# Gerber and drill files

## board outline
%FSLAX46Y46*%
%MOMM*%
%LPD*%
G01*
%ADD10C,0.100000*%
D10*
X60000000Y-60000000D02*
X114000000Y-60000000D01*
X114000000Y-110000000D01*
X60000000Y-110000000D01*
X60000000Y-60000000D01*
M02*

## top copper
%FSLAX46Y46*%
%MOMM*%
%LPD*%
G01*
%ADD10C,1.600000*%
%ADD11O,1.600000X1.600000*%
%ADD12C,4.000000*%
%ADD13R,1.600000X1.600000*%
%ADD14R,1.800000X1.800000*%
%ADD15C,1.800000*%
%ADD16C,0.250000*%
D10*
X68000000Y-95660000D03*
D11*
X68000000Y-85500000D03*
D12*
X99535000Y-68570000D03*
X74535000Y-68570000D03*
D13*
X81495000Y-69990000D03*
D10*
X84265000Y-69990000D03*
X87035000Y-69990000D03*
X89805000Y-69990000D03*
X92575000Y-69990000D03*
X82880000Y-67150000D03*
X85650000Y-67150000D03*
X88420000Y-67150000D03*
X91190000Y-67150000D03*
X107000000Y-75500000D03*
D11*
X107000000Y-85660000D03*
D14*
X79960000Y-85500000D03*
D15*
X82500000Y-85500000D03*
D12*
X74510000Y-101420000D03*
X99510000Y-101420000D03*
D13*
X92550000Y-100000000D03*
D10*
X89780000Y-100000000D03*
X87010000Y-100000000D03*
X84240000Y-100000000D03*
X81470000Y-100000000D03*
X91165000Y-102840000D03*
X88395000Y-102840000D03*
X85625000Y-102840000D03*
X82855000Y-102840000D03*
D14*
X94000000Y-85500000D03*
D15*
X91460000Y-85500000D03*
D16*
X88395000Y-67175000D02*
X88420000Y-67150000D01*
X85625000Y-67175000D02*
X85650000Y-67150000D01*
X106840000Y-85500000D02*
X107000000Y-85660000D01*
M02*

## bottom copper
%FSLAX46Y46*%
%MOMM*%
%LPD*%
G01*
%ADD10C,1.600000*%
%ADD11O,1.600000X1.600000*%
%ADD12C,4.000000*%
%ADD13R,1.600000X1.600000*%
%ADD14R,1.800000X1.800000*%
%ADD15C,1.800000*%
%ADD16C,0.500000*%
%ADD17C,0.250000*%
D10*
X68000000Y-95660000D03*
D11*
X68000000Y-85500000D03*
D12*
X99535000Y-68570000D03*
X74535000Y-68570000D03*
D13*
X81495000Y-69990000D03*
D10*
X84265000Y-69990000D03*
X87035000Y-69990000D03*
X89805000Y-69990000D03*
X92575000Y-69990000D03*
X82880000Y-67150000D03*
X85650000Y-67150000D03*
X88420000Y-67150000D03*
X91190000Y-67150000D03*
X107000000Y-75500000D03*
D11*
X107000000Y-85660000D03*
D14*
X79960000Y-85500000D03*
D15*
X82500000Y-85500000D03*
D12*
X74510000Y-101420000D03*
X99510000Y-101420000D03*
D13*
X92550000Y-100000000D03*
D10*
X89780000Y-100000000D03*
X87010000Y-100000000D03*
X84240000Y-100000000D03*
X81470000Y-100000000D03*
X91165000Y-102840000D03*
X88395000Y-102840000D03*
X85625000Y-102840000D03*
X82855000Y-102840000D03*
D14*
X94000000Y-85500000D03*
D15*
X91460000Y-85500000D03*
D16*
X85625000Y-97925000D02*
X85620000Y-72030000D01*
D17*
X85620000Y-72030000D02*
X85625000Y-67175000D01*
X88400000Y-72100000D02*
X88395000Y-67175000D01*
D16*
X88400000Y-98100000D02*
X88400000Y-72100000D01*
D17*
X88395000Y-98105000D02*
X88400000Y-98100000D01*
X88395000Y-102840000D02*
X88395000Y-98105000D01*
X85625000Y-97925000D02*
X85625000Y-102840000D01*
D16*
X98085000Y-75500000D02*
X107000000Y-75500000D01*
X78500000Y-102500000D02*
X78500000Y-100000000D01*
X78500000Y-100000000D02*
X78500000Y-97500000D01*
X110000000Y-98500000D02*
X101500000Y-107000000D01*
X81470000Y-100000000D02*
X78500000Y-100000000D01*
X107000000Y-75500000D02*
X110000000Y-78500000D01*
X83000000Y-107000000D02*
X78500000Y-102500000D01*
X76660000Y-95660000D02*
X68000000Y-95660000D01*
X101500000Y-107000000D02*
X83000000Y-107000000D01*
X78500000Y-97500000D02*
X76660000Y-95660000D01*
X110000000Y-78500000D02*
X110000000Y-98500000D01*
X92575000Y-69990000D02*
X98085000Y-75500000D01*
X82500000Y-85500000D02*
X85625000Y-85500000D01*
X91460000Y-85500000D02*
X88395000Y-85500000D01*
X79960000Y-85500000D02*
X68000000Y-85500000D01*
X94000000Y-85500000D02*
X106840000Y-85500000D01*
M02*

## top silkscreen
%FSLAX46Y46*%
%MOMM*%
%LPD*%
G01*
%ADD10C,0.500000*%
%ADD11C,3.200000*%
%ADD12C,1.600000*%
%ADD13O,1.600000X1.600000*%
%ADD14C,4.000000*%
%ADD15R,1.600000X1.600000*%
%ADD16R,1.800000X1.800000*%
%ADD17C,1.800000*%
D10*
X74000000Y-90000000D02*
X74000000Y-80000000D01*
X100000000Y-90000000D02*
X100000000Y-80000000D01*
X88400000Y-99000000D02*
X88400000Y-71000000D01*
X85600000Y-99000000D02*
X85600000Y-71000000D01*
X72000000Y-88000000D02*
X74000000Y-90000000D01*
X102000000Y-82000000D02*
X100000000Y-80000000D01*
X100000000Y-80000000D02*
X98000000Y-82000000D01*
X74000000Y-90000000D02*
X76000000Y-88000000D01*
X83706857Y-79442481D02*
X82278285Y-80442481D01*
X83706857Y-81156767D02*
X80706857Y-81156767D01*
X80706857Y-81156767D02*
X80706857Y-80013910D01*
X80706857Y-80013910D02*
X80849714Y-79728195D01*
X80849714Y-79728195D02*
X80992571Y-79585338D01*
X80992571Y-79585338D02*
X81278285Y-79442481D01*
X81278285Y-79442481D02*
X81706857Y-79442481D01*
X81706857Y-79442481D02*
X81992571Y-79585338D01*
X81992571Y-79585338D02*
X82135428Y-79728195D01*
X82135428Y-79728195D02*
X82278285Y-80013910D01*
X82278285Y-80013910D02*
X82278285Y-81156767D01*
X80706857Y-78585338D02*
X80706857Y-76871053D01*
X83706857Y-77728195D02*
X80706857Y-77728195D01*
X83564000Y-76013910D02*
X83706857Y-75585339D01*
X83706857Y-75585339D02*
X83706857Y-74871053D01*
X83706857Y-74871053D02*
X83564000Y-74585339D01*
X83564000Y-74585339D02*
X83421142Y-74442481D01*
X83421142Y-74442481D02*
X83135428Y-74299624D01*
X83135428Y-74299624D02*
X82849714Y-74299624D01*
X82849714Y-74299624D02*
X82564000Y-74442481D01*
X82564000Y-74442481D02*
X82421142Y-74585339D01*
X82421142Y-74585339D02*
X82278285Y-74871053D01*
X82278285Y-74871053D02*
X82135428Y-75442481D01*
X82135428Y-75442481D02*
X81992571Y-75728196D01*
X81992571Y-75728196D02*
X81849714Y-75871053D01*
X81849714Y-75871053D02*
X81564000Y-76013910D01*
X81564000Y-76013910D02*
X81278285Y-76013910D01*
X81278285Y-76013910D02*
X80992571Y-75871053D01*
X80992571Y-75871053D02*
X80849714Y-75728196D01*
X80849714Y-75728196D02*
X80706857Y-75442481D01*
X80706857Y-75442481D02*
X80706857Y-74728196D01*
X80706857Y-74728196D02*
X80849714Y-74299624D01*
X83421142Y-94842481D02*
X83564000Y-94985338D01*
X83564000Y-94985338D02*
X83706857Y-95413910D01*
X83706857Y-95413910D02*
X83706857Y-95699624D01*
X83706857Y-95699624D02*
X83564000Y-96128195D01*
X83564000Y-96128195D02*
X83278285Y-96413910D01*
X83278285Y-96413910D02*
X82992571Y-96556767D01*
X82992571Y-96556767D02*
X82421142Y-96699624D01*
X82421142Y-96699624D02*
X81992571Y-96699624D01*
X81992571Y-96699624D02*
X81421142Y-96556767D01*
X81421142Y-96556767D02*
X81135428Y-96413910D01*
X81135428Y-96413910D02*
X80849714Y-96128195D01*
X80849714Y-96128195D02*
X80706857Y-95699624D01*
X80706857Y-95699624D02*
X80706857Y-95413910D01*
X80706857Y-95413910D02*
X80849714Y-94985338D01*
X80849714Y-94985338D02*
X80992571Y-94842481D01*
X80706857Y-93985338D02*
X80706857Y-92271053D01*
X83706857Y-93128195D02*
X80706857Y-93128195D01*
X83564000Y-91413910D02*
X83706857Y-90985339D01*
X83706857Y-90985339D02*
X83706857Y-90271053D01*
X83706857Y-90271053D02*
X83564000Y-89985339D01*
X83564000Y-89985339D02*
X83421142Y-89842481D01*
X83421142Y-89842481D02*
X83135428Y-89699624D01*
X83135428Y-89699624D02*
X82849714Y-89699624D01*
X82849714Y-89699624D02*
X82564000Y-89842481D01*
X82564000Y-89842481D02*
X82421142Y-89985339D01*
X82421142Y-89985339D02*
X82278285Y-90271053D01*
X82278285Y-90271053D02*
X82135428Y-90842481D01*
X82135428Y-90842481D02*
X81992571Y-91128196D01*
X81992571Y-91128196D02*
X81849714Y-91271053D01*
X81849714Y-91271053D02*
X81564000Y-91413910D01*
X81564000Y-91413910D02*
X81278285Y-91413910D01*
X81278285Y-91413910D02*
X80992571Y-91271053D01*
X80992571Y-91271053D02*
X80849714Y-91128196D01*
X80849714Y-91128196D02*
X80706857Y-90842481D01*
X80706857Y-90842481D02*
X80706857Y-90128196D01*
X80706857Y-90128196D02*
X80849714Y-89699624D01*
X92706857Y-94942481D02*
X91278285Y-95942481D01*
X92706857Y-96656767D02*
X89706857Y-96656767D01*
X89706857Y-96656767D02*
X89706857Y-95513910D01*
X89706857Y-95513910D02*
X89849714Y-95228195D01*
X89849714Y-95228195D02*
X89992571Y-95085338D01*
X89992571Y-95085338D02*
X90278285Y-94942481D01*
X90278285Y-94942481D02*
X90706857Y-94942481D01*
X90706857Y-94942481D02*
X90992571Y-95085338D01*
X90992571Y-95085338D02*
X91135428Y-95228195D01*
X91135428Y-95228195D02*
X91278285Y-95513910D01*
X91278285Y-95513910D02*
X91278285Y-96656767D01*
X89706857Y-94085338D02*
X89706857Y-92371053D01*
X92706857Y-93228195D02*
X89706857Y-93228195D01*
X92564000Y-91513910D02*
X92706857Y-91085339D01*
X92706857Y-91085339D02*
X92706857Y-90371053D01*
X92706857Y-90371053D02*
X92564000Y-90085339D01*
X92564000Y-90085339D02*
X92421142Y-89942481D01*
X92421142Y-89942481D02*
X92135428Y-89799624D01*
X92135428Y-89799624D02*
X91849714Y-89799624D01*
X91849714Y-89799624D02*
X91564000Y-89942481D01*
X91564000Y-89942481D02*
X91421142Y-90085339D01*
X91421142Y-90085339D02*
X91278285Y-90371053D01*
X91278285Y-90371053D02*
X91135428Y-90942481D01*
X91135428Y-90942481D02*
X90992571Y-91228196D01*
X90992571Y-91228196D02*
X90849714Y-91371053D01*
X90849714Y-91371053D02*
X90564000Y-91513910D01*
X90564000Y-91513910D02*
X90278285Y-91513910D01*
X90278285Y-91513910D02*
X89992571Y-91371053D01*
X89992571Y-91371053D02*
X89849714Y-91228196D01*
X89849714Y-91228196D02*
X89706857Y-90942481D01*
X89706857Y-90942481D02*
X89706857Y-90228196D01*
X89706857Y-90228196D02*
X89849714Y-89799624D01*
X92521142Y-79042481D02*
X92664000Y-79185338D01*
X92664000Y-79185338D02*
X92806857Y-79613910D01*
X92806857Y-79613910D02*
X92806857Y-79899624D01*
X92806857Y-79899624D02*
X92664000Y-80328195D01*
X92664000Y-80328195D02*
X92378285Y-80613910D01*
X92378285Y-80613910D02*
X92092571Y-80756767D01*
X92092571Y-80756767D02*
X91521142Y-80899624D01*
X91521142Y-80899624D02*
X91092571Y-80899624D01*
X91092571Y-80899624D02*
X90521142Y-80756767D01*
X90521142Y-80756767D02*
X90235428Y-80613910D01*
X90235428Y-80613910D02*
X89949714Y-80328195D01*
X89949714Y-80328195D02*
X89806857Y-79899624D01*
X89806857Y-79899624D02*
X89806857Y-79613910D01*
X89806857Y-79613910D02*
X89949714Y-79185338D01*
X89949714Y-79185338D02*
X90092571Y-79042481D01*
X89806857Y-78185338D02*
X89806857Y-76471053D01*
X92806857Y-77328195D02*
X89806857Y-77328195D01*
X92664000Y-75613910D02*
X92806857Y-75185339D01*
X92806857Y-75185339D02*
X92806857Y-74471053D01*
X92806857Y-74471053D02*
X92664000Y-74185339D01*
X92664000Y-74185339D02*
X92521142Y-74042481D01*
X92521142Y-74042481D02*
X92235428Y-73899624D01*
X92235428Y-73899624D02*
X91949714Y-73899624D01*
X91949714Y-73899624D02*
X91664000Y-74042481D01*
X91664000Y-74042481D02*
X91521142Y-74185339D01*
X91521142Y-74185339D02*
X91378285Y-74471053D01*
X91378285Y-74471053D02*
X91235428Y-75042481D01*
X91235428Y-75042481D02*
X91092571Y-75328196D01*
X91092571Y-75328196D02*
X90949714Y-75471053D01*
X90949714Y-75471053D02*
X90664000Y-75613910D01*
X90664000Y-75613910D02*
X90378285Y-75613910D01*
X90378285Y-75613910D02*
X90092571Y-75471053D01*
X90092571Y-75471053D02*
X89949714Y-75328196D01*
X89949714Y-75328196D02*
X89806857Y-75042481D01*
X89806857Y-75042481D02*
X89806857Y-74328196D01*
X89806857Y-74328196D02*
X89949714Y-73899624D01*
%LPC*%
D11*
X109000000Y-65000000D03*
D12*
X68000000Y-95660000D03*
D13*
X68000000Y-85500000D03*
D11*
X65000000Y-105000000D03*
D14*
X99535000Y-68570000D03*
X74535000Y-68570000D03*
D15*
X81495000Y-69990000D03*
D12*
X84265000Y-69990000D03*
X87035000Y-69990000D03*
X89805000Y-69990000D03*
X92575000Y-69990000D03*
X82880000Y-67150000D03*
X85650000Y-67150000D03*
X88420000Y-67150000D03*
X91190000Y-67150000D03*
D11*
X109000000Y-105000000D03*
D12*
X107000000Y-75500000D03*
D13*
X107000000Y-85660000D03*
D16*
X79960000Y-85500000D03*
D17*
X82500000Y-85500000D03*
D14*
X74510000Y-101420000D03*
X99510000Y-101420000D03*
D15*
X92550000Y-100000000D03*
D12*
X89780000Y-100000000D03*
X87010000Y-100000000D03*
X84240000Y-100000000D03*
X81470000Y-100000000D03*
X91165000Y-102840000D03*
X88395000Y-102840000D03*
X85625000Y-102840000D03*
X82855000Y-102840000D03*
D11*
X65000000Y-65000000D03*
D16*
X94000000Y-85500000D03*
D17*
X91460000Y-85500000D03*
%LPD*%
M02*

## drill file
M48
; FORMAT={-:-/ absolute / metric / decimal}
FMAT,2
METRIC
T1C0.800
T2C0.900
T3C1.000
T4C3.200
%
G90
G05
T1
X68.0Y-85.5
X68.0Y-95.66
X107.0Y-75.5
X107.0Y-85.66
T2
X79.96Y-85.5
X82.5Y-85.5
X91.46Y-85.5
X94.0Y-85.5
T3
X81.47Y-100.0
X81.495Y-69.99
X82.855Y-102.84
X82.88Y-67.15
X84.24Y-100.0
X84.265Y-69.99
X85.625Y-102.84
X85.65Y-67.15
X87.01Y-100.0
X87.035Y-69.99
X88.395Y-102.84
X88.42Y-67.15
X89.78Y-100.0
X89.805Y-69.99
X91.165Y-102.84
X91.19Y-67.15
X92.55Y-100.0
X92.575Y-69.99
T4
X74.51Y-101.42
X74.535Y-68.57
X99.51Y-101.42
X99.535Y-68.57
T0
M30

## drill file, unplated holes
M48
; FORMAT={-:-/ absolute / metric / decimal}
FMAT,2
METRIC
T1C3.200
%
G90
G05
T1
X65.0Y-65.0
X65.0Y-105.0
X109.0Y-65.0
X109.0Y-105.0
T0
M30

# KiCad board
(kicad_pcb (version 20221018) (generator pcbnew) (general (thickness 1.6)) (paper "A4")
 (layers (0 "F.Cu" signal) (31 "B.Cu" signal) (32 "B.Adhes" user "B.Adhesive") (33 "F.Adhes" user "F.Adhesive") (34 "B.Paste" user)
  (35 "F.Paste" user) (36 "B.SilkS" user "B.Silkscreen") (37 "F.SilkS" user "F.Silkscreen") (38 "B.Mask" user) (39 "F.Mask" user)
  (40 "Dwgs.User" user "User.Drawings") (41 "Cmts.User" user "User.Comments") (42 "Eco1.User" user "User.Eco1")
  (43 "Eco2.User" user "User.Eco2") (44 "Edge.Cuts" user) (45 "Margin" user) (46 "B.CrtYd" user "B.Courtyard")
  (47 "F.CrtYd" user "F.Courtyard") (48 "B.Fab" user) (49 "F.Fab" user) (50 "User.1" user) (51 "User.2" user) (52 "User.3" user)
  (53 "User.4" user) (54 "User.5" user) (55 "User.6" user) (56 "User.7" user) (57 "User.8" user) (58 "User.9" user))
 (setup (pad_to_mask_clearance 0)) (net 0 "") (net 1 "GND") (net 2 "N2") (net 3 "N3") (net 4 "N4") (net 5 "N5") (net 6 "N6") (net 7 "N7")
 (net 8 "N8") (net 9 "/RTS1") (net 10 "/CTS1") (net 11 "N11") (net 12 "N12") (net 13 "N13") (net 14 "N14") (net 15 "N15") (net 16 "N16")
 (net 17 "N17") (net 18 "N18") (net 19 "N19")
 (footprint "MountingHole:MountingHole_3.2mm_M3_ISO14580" (layer "F.Cu") (at 109 65)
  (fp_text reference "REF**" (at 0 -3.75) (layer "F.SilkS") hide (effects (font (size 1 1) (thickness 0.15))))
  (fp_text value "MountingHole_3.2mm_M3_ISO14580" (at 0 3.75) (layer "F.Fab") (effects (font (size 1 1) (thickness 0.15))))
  (pad "" np_thru_hole circle (at 0 0) (size 3.2 3.2) (drill 3.2) (layers "*.Cu" "*.Mask")))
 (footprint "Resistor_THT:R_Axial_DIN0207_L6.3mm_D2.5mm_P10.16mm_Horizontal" (layer "F.Cu") (at 68 95.66 90)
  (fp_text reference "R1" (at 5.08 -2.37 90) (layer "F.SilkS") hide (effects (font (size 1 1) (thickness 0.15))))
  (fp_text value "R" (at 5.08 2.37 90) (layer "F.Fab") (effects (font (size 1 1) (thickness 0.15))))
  (pad "1" thru_hole circle (at 0 0 90) (size 1.6 1.6) (drill 0.8) (layers "*.Cu" "*.Mask") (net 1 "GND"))
  (pad "2" thru_hole oval (at 10.16 0 90) (size 1.6 1.6) (drill 0.8) (layers "*.Cu" "*.Mask") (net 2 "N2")))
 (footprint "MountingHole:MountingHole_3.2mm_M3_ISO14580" (layer "F.Cu") (at 65 105)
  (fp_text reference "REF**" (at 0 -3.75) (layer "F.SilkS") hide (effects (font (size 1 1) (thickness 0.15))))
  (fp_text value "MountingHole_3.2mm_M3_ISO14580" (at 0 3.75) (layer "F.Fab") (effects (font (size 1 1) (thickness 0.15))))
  (pad "" np_thru_hole circle (at 0 0) (size 3.2 3.2) (drill 3.2) (layers "*.Cu" "*.Mask")))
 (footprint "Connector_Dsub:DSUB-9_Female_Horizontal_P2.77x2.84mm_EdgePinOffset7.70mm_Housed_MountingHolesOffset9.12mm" (layer "F.Cu")
  (at 81.495 69.99 180)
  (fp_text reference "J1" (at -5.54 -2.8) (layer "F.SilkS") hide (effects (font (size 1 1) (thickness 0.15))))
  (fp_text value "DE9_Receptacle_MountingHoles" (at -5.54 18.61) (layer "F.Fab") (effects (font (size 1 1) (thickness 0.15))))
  (pad "0" thru_hole circle (at -18.04 1.42 180) (size 4 4) (drill 3.2) (layers "*.Cu" "*.Mask") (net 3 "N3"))
  (pad "0" thru_hole circle (at 6.96 1.42 180) (size 4 4) (drill 3.2) (layers "*.Cu" "*.Mask") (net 3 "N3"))
  (pad "1" thru_hole rect (at 0 0 180) (size 1.6 1.6) (drill 1) (layers "*.Cu" "*.Mask") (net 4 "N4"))
  (pad "2" thru_hole circle (at -2.77 0 180) (size 1.6 1.6) (drill 1) (layers "*.Cu" "*.Mask") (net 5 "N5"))
  (pad "3" thru_hole circle (at -5.54 0 180) (size 1.6 1.6) (drill 1) (layers "*.Cu" "*.Mask") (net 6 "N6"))
  (pad "4" thru_hole circle (at -8.31 0 180) (size 1.6 1.6) (drill 1) (layers "*.Cu" "*.Mask") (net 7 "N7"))
  (pad "5" thru_hole circle (at -11.08 0 180) (size 1.6 1.6) (drill 1) (layers "*.Cu" "*.Mask") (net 1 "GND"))
  (pad "6" thru_hole circle (at -1.385 2.84 180) (size 1.6 1.6) (drill 1) (layers "*.Cu" "*.Mask") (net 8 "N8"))
  (pad "7" thru_hole circle (at -4.155 2.84 180) (size 1.6 1.6) (drill 1) (layers "*.Cu" "*.Mask") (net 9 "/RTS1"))
  (pad "8" thru_hole circle (at -6.925 2.84 180) (size 1.6 1.6) (drill 1) (layers "*.Cu" "*.Mask") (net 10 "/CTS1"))
  (pad "9" thru_hole circle (at -9.695 2.84 180) (size 1.6 1.6) (drill 1) (layers "*.Cu" "*.Mask") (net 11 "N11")))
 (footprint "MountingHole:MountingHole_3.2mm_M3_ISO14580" (layer "F.Cu") (at 109 105)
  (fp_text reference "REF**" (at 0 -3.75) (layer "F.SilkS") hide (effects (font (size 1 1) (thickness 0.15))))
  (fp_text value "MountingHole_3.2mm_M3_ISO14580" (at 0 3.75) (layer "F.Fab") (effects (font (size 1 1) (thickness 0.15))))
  (pad "" np_thru_hole circle (at 0 0) (size 3.2 3.2) (drill 3.2) (layers "*.Cu" "*.Mask")))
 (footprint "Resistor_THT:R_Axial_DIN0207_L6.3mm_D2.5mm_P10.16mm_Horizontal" (layer "F.Cu") (at 107 75.5 -90)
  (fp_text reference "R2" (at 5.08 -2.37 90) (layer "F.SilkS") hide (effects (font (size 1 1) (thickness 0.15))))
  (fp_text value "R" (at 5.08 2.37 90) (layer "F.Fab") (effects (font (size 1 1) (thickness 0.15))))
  (pad "1" thru_hole circle (at 0 0 270) (size 1.6 1.6) (drill 0.8) (layers "*.Cu" "*.Mask") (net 1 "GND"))
  (pad "2" thru_hole oval (at 10.16 0 270) (size 1.6 1.6) (drill 0.8) (layers "*.Cu" "*.Mask") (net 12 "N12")))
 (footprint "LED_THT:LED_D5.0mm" (layer "F.Cu") (at 79.96 85.5)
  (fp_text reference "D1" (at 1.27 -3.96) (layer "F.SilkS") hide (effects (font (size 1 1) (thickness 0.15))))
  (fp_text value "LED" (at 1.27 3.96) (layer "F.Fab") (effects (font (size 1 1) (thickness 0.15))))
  (pad "1" thru_hole rect (at 0 0) (size 1.8 1.8) (drill 0.9) (layers "*.Cu" "*.Mask") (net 2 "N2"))
  (pad "2" thru_hole circle (at 2.54 0) (size 1.8 1.8) (drill 0.9) (layers "*.Cu" "*.Mask") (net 9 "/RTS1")))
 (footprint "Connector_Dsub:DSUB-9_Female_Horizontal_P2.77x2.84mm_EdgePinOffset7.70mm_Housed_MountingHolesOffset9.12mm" (layer "F.Cu")
  (at 92.55 100)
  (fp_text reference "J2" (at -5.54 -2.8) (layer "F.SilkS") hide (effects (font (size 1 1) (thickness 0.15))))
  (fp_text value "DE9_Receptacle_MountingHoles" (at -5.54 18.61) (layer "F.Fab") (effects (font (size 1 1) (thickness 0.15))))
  (pad "0" thru_hole circle (at -18.04 1.42) (size 4 4) (drill 3.2) (layers "*.Cu" "*.Mask") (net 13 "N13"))
  (pad "0" thru_hole circle (at 6.96 1.42) (size 4 4) (drill 3.2) (layers "*.Cu" "*.Mask") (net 13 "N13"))
  (pad "1" thru_hole rect (at 0 0) (size 1.6 1.6) (drill 1) (layers "*.Cu" "*.Mask") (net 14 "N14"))
  (pad "2" thru_hole circle (at -2.77 0) (size 1.6 1.6) (drill 1) (layers "*.Cu" "*.Mask") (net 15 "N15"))
  (pad "3" thru_hole circle (at -5.54 0) (size 1.6 1.6) (drill 1) (layers "*.Cu" "*.Mask") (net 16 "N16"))
  (pad "4" thru_hole circle (at -8.31 0) (size 1.6 1.6) (drill 1) (layers "*.Cu" "*.Mask") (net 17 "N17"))
  (pad "5" thru_hole circle (at -11.08 0) (size 1.6 1.6) (drill 1) (layers "*.Cu" "*.Mask") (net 1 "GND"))
  (pad "6" thru_hole circle (at -1.385 2.84) (size 1.6 1.6) (drill 1) (layers "*.Cu" "*.Mask") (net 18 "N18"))
  (pad "7" thru_hole circle (at -4.155 2.84) (size 1.6 1.6) (drill 1) (layers "*.Cu" "*.Mask") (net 10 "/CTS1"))
  (pad "8" thru_hole circle (at -6.925 2.84) (size 1.6 1.6) (drill 1) (layers "*.Cu" "*.Mask") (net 9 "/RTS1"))
  (pad "9" thru_hole circle (at -9.695 2.84) (size 1.6 1.6) (drill 1) (layers "*.Cu" "*.Mask") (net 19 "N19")))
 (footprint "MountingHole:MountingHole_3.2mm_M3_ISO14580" (layer "F.Cu") (at 65 65)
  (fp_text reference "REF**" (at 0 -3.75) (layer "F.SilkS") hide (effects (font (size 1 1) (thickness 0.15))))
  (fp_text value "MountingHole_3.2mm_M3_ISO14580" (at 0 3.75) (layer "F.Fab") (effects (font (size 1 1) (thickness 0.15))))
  (pad "" np_thru_hole circle (at 0 0) (size 3.2 3.2) (drill 3.2) (layers "*.Cu" "*.Mask")))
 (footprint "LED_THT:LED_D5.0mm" (layer "F.Cu") (at 94 85.5 180)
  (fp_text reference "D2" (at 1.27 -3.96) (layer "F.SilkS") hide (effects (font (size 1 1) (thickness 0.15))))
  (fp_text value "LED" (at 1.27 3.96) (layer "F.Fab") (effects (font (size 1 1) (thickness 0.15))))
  (pad "1" thru_hole rect (at 0 0 180) (size 1.8 1.8) (drill 0.9) (layers "*.Cu" "*.Mask") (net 12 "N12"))
  (pad "2" thru_hole circle (at 2.54 0 180) (size 1.8 1.8) (drill 0.9) (layers "*.Cu" "*.Mask") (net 10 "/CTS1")))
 (gr_line (start 74 90) (end 74 80) (stroke (width 0.5) (type default)) (layer "F.SilkS"))
 (gr_line (start 100 90) (end 100 80) (stroke (width 0.5) (type default)) (layer "F.SilkS"))
 (gr_line (start 88.4 99) (end 88.4 71) (stroke (width 0.5) (type default)) (layer "F.SilkS"))
 (gr_line (start 85.6 99) (end 85.6 71) (stroke (width 0.5) (type default)) (layer "F.SilkS"))
 (gr_line (start 72 88) (end 74 90) (stroke (width 0.5) (type default)) (layer "F.SilkS"))
 (gr_line (start 102 82) (end 100 80) (stroke (width 0.5) (type default)) (layer "F.SilkS"))
 (gr_line (start 100 80) (end 98 82) (stroke (width 0.5) (type default)) (layer "F.SilkS"))
 (gr_line (start 74 90) (end 76 88) (stroke (width 0.5) (type default)) (layer "F.SilkS"))
 (gr_rect (start 60 60) (end 114 110) (stroke (width 0.1) (type default)) (fill none) (layer "Edge.Cuts"))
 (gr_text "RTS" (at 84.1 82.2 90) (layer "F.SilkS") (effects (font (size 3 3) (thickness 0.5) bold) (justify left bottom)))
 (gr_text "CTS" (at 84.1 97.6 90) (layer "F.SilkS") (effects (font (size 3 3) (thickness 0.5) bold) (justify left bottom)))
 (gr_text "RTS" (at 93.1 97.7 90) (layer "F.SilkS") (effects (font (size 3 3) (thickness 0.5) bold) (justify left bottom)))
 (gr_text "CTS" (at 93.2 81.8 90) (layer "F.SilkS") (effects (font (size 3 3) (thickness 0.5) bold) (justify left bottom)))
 (segment (start 98.085 75.5) (end 107 75.5) (width 0.5) (layer "B.Cu") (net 1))
 (segment (start 78.5 102.5) (end 78.5 100) (width 0.5) (layer "B.Cu") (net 1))
 (segment (start 78.5 100) (end 78.5 97.5) (width 0.5) (layer "B.Cu") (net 1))
 (segment (start 110 98.5) (end 101.5 107) (width 0.5) (layer "B.Cu") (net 1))
 (segment (start 81.47 100) (end 78.5 100) (width 0.5) (layer "B.Cu") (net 1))
 (segment (start 107 75.5) (end 110 78.5) (width 0.5) (layer "B.Cu") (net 1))
 (segment (start 83 107) (end 78.5 102.5) (width 0.5) (layer "B.Cu") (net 1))
 (segment (start 76.66 95.66) (end 68 95.66) (width 0.5) (layer "B.Cu") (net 1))
 (segment (start 101.5 107) (end 83 107) (width 0.5) (layer "B.Cu") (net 1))
 (segment (start 78.5 97.5) (end 76.66 95.66) (width 0.5) (layer "B.Cu") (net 1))
 (segment (start 110 78.5) (end 110 98.5) (width 0.5) (layer "B.Cu") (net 1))
 (segment (start 92.575 69.99) (end 98.085 75.5) (width 0.5) (layer "B.Cu") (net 1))
 (segment (start 85.625 67.175) (end 85.65 67.15) (width 0.25) (layer "F.Cu") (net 9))
 (segment (start 85.62 72.03) (end 85.625 67.175) (width 0.25) (layer "B.Cu") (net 9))
 (segment (start 85.625 97.925) (end 85.625 102.84) (width 0.25) (layer "B.Cu") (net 9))
 (segment (start 85.625 97.925) (end 85.62 72.03) (width 0.5) (layer "B.Cu") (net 9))
 (segment (start 82.5 85.5) (end 85.625 85.5) (width 0.5) (layer "B.Cu") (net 9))
 (segment (start 88.395 67.175) (end 88.42 67.15) (width 0.25) (layer "F.Cu") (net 10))
 (segment (start 88.4 72.1) (end 88.395 67.175) (width 0.25) (layer "B.Cu") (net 10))
 (segment (start 88.395 102.84) (end 88.395 98.105) (width 0.25) (layer "B.Cu") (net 10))
 (segment (start 91.46 85.5) (end 88.395 85.5) (width 0.5) (layer "B.Cu") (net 10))
 (segment (start 88.395 98.105) (end 88.4 98.1) (width 0.25) (layer "B.Cu") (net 10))
 (segment (start 88.4 98.1) (end 88.4 72.1) (width 0.5) (layer "B.Cu") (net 10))
 (segment (start 79.96 85.5) (end 68 85.5) (width 0.5) (layer "B.Cu") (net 2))
 (segment (start 106.84 85.5) (end 107 85.66) (width 0.25) (layer "F.Cu") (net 12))
 (segment (start 94 85.5) (end 106.84 85.5) (width 0.5) (layer "B.Cu") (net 12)))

